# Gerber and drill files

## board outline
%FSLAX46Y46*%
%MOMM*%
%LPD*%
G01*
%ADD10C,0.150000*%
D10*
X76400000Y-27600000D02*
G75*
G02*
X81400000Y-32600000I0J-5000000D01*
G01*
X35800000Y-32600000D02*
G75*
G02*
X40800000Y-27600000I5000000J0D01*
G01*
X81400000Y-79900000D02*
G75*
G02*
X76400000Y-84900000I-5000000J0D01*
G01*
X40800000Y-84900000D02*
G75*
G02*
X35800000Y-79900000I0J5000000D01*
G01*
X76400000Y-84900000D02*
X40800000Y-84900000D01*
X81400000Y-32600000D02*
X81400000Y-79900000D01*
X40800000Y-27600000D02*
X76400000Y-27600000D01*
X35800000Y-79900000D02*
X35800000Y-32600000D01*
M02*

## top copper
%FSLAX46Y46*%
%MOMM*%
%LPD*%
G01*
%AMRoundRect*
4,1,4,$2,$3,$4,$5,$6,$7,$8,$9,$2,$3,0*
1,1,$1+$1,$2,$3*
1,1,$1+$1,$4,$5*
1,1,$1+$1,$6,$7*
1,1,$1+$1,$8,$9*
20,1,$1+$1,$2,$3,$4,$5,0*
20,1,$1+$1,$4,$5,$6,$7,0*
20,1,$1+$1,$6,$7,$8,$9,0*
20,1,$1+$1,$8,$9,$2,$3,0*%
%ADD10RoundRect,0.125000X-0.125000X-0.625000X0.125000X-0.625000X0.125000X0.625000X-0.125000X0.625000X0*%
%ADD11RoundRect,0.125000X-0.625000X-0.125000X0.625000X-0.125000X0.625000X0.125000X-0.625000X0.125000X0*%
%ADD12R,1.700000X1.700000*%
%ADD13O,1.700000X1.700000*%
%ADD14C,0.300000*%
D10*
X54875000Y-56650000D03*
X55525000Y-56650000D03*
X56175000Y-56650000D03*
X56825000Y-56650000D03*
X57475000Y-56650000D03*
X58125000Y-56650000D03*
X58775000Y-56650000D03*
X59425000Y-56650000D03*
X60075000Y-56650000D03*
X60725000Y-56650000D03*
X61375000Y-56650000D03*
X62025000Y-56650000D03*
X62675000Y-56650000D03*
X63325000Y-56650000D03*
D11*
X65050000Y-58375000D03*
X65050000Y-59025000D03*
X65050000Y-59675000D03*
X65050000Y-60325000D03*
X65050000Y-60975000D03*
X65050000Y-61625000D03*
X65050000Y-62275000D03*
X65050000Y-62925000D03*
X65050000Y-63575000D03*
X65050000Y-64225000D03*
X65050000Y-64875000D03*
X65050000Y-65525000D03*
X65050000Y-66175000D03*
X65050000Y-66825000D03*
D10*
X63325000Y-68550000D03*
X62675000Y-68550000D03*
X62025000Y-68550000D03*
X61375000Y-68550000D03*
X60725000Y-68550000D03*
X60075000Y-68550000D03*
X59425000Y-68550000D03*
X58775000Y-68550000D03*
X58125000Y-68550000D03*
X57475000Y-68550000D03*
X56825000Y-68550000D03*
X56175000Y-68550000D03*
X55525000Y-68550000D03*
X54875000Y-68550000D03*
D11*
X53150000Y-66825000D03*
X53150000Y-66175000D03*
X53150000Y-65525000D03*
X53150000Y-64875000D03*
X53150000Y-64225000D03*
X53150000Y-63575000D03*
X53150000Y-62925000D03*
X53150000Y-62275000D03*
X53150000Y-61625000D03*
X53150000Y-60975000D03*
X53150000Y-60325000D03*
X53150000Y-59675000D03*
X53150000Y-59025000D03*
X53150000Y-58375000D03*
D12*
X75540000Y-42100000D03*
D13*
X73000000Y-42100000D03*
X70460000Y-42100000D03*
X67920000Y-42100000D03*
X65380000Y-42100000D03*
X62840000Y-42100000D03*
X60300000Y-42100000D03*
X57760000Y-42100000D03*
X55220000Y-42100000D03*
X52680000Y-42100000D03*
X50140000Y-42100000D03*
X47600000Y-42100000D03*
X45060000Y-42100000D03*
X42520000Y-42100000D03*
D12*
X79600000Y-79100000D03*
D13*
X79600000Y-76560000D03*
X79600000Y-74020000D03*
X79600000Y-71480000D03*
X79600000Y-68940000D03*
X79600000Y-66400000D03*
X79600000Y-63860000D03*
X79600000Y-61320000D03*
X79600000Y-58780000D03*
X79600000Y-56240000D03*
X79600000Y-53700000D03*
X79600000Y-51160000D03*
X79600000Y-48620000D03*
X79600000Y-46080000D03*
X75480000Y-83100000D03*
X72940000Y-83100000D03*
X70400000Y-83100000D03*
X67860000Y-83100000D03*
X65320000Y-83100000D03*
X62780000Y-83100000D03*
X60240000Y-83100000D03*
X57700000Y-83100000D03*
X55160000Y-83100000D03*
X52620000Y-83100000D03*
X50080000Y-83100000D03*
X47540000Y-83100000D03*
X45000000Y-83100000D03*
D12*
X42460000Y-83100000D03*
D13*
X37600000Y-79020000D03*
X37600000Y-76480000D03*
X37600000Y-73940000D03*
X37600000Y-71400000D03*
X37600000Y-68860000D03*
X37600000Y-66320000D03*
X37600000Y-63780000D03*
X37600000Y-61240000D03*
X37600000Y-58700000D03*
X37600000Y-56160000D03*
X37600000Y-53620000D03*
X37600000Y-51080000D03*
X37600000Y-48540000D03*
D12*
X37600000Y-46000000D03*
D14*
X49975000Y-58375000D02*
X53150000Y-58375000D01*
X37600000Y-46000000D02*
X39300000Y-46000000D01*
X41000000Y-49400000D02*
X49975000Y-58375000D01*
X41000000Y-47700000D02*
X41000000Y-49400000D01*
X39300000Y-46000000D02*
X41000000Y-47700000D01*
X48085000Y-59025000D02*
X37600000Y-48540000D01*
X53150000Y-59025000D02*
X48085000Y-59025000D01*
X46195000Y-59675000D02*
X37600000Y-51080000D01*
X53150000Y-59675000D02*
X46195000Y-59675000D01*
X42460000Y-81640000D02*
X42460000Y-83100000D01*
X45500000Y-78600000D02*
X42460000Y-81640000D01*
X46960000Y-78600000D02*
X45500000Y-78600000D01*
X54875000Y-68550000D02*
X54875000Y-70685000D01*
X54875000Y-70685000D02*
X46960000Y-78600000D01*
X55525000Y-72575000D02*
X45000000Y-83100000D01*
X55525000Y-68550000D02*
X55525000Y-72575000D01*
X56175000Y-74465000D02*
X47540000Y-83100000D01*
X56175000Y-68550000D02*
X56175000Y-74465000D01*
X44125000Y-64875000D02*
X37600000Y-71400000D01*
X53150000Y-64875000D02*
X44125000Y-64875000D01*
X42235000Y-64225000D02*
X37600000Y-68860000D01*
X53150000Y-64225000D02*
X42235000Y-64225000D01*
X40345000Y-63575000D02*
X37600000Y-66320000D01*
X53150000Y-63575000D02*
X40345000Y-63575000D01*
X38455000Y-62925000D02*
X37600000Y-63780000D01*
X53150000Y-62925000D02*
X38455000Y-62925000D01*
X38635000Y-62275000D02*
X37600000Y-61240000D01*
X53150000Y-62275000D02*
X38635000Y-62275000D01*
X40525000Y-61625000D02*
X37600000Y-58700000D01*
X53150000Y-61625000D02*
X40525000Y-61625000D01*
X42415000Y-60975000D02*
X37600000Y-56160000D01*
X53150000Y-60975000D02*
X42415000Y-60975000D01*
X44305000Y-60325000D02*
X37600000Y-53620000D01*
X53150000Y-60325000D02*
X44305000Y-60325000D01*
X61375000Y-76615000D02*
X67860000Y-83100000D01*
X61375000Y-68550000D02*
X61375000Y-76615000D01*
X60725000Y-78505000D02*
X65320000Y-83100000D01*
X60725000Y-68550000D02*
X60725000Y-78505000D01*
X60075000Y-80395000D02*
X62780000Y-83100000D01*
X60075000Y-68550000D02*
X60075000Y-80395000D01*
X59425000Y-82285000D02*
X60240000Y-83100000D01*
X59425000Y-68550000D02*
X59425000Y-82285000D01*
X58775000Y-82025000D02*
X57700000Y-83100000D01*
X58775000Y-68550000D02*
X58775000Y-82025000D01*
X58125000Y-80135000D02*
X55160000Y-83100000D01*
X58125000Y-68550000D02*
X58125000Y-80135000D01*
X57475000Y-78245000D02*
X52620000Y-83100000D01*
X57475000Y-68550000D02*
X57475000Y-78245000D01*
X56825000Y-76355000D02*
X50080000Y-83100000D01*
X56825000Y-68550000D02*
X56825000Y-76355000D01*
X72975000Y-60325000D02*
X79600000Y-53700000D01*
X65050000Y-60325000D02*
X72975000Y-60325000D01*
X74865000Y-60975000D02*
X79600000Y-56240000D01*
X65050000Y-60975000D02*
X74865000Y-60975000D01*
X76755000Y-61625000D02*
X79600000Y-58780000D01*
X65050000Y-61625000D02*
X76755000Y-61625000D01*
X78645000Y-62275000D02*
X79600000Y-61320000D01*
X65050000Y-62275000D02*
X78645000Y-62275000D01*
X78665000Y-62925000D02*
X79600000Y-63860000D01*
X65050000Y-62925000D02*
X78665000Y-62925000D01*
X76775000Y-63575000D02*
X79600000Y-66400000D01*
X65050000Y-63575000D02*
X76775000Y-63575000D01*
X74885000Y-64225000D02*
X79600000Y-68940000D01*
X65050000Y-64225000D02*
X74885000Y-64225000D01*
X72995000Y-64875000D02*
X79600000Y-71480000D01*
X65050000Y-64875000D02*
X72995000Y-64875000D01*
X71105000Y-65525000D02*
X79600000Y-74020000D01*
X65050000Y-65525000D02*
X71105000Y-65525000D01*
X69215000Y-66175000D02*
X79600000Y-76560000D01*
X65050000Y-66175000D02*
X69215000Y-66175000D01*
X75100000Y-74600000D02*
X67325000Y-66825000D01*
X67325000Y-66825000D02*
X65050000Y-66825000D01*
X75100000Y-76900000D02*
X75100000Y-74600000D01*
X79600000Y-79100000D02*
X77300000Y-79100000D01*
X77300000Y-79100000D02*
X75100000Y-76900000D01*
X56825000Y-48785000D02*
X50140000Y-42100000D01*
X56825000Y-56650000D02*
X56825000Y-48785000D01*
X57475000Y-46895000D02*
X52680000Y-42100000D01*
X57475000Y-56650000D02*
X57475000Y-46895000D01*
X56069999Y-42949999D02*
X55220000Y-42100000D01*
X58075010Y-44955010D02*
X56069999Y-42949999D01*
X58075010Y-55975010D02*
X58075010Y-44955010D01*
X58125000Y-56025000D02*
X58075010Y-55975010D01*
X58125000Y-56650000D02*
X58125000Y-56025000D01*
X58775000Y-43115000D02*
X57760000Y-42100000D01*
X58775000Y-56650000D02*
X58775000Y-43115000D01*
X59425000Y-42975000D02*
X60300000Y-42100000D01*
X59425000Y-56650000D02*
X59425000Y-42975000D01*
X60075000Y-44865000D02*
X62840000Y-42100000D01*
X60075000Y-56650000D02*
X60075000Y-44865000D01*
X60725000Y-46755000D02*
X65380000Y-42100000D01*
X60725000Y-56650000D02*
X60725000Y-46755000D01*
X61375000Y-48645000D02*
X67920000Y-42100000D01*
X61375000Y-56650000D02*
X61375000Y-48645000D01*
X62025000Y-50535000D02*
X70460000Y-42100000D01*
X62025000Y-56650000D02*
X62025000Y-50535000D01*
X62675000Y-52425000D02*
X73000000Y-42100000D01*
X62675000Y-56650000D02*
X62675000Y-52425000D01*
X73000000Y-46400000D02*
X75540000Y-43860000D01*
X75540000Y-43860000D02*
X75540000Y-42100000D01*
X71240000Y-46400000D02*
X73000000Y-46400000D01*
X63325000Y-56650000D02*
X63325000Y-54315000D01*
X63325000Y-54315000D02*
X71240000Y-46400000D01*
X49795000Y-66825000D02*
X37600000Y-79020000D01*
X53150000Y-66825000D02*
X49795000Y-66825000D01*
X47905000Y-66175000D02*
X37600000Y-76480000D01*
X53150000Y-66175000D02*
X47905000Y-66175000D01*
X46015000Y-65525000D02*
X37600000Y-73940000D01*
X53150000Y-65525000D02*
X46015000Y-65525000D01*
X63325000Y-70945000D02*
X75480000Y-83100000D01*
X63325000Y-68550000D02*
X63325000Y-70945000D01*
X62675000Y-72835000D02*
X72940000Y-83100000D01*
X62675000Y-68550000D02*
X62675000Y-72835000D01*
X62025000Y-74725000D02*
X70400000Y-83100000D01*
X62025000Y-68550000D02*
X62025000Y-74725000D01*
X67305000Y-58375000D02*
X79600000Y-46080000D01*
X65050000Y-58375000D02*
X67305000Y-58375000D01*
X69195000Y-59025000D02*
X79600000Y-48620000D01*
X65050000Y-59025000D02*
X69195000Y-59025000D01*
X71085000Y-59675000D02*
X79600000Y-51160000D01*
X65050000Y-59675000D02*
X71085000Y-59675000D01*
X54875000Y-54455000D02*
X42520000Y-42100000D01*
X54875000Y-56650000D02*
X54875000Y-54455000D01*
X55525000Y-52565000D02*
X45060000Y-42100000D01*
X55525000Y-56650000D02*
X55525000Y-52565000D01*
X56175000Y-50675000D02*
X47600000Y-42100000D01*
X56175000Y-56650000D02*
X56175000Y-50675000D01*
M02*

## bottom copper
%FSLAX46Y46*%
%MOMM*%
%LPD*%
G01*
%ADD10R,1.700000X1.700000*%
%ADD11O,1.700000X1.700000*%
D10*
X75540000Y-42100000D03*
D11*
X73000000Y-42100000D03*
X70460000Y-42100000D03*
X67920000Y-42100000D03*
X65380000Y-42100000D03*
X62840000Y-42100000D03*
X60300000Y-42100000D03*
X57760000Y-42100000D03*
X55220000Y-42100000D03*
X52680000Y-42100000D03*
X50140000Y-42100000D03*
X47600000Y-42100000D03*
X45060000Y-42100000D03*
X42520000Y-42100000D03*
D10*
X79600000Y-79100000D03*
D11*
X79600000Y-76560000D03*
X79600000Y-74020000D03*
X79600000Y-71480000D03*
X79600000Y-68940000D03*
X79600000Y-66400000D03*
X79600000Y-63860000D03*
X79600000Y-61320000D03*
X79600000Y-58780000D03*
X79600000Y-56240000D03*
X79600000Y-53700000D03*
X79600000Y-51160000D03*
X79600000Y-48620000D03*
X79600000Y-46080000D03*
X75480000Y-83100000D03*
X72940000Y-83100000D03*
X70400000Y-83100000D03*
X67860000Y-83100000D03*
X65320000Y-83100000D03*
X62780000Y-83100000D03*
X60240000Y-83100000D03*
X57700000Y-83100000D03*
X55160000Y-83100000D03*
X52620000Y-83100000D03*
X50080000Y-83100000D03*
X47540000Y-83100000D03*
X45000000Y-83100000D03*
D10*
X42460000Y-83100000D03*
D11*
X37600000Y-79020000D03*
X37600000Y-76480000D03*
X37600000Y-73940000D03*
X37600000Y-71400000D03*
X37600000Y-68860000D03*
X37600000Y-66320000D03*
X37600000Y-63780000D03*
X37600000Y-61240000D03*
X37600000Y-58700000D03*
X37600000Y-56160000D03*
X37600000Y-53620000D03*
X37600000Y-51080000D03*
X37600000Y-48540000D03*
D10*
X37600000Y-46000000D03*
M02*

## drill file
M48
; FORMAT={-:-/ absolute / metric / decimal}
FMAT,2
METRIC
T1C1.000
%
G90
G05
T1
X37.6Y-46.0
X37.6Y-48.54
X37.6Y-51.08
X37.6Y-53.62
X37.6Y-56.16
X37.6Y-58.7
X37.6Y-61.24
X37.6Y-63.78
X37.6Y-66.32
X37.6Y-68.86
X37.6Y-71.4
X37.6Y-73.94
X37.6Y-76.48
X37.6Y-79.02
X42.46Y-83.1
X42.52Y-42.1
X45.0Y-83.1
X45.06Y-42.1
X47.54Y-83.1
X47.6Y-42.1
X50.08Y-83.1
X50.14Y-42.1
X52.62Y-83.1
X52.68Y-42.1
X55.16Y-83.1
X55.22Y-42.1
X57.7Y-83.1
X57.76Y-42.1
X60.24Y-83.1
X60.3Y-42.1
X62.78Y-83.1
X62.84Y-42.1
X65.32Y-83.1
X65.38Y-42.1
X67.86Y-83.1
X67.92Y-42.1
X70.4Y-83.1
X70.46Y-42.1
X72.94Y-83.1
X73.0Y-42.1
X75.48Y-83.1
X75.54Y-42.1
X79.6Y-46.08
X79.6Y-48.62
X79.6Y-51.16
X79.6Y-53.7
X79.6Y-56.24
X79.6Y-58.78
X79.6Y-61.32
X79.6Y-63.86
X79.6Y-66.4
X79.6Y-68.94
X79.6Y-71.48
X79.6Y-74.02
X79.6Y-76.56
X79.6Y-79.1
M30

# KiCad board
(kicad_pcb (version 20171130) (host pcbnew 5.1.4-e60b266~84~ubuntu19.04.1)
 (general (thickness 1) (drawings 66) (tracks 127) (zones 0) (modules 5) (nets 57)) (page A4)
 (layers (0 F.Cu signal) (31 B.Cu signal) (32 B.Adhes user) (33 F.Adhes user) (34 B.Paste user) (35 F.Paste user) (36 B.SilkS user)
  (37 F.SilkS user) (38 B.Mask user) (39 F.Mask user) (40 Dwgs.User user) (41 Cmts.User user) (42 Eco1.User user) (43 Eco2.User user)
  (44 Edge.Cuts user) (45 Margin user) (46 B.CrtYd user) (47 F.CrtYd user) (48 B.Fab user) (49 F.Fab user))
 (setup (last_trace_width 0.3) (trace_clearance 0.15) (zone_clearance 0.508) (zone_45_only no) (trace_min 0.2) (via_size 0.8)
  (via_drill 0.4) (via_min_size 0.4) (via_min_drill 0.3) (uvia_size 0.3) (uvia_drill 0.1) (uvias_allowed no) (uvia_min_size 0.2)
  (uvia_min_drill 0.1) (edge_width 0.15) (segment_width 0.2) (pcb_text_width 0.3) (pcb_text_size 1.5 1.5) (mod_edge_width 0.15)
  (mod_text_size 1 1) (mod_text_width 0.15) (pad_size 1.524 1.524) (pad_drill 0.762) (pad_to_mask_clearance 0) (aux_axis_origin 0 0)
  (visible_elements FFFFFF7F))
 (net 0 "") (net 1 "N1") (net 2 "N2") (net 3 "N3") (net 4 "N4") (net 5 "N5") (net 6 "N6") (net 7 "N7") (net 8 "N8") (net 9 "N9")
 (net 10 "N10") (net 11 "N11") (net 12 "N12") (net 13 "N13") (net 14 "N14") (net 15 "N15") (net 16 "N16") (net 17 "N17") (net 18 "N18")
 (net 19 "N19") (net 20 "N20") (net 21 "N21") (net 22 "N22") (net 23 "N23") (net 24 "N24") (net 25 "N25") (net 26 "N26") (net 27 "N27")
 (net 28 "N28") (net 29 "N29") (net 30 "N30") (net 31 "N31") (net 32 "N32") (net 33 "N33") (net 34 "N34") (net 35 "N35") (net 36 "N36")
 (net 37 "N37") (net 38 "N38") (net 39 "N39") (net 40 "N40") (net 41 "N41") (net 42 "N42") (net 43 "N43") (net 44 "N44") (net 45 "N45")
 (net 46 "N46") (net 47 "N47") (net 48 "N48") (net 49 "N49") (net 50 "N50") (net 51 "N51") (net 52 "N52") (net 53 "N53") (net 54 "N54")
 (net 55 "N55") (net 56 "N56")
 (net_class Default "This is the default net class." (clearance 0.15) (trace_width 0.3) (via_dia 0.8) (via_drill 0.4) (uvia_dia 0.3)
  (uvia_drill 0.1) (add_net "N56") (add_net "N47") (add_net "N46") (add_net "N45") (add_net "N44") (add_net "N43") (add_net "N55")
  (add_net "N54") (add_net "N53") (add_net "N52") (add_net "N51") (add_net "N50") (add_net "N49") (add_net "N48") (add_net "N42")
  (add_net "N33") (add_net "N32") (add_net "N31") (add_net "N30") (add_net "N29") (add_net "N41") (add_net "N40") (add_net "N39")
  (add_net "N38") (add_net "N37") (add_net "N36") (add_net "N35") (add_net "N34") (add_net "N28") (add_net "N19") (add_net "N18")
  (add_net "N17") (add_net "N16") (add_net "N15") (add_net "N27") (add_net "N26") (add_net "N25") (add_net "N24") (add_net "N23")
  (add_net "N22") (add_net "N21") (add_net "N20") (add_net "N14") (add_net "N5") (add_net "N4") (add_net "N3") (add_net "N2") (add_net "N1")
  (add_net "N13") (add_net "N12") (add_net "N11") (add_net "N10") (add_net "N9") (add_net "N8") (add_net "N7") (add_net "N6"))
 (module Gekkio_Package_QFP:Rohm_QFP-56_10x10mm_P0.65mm (layer F.Cu) (at 59.1 62.6)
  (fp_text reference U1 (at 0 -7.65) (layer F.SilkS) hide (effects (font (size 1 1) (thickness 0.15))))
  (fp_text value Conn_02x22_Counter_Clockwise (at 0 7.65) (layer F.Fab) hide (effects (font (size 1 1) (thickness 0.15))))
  (pad 56 smd roundrect (at -4.225 -5.95) (size 0.5 1.5) (layers F.Cu F.Paste F.Mask) (roundrect_rratio 0.25) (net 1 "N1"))
  (pad 55 smd roundrect (at -3.575 -5.95) (size 0.5 1.5) (layers F.Cu F.Paste F.Mask) (roundrect_rratio 0.25) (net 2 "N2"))
  (pad 54 smd roundrect (at -2.925 -5.95) (size 0.5 1.5) (layers F.Cu F.Paste F.Mask) (roundrect_rratio 0.25) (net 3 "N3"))
  (pad 53 smd roundrect (at -2.275 -5.95) (size 0.5 1.5) (layers F.Cu F.Paste F.Mask) (roundrect_rratio 0.25) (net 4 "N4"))
  (pad 52 smd roundrect (at -1.625 -5.95) (size 0.5 1.5) (layers F.Cu F.Paste F.Mask) (roundrect_rratio 0.25) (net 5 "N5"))
  (pad 51 smd roundrect (at -0.975 -5.95) (size 0.5 1.5) (layers F.Cu F.Paste F.Mask) (roundrect_rratio 0.25) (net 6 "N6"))
  (pad 50 smd roundrect (at -0.325 -5.95) (size 0.5 1.5) (layers F.Cu F.Paste F.Mask) (roundrect_rratio 0.25) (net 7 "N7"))
  (pad 49 smd roundrect (at 0.325 -5.95) (size 0.5 1.5) (layers F.Cu F.Paste F.Mask) (roundrect_rratio 0.25) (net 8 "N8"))
  (pad 48 smd roundrect (at 0.975 -5.95) (size 0.5 1.5) (layers F.Cu F.Paste F.Mask) (roundrect_rratio 0.25) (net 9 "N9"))
  (pad 47 smd roundrect (at 1.625 -5.95) (size 0.5 1.5) (layers F.Cu F.Paste F.Mask) (roundrect_rratio 0.25) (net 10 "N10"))
  (pad 46 smd roundrect (at 2.275 -5.95) (size 0.5 1.5) (layers F.Cu F.Paste F.Mask) (roundrect_rratio 0.25) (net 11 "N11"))
  (pad 45 smd roundrect (at 2.925 -5.95) (size 0.5 1.5) (layers F.Cu F.Paste F.Mask) (roundrect_rratio 0.25) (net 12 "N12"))
  (pad 44 smd roundrect (at 3.575 -5.95) (size 0.5 1.5) (layers F.Cu F.Paste F.Mask) (roundrect_rratio 0.25) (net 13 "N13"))
  (pad 43 smd roundrect (at 4.225 -5.95) (size 0.5 1.5) (layers F.Cu F.Paste F.Mask) (roundrect_rratio 0.25) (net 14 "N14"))
  (pad 42 smd roundrect (at 5.95 -4.225) (size 1.5 0.5) (layers F.Cu F.Paste F.Mask) (roundrect_rratio 0.25) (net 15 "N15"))
  (pad 41 smd roundrect (at 5.95 -3.575) (size 1.5 0.5) (layers F.Cu F.Paste F.Mask) (roundrect_rratio 0.25) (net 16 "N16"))
  (pad 40 smd roundrect (at 5.95 -2.925) (size 1.5 0.5) (layers F.Cu F.Paste F.Mask) (roundrect_rratio 0.25) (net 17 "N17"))
  (pad 39 smd roundrect (at 5.95 -2.275) (size 1.5 0.5) (layers F.Cu F.Paste F.Mask) (roundrect_rratio 0.25) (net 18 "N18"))
  (pad 38 smd roundrect (at 5.95 -1.625) (size 1.5 0.5) (layers F.Cu F.Paste F.Mask) (roundrect_rratio 0.25) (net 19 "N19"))
  (pad 37 smd roundrect (at 5.95 -0.975) (size 1.5 0.5) (layers F.Cu F.Paste F.Mask) (roundrect_rratio 0.25) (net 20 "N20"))
  (pad 36 smd roundrect (at 5.95 -0.325) (size 1.5 0.5) (layers F.Cu F.Paste F.Mask) (roundrect_rratio 0.25) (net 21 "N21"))
  (pad 35 smd roundrect (at 5.95 0.325) (size 1.5 0.5) (layers F.Cu F.Paste F.Mask) (roundrect_rratio 0.25) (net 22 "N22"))
  (pad 34 smd roundrect (at 5.95 0.975) (size 1.5 0.5) (layers F.Cu F.Paste F.Mask) (roundrect_rratio 0.25) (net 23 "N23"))
  (pad 33 smd roundrect (at 5.95 1.625) (size 1.5 0.5) (layers F.Cu F.Paste F.Mask) (roundrect_rratio 0.25) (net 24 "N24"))
  (pad 32 smd roundrect (at 5.95 2.275) (size 1.5 0.5) (layers F.Cu F.Paste F.Mask) (roundrect_rratio 0.25) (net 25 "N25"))
  (pad 31 smd roundrect (at 5.95 2.925) (size 1.5 0.5) (layers F.Cu F.Paste F.Mask) (roundrect_rratio 0.25) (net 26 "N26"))
  (pad 30 smd roundrect (at 5.95 3.575) (size 1.5 0.5) (layers F.Cu F.Paste F.Mask) (roundrect_rratio 0.25) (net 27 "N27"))
  (pad 29 smd roundrect (at 5.95 4.225) (size 1.5 0.5) (layers F.Cu F.Paste F.Mask) (roundrect_rratio 0.25) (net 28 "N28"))
  (pad 28 smd roundrect (at 4.225 5.95) (size 0.5 1.5) (layers F.Cu F.Paste F.Mask) (roundrect_rratio 0.25) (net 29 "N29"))
  (pad 27 smd roundrect (at 3.575 5.95) (size 0.5 1.5) (layers F.Cu F.Paste F.Mask) (roundrect_rratio 0.25) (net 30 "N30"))
  (pad 26 smd roundrect (at 2.925 5.95) (size 0.5 1.5) (layers F.Cu F.Paste F.Mask) (roundrect_rratio 0.25) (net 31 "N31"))
  (pad 25 smd roundrect (at 2.275 5.95) (size 0.5 1.5) (layers F.Cu F.Paste F.Mask) (roundrect_rratio 0.25) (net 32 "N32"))
  (pad 24 smd roundrect (at 1.625 5.95) (size 0.5 1.5) (layers F.Cu F.Paste F.Mask) (roundrect_rratio 0.25) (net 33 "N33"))
  (pad 23 smd roundrect (at 0.975 5.95) (size 0.5 1.5) (layers F.Cu F.Paste F.Mask) (roundrect_rratio 0.25) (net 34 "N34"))
  (pad 22 smd roundrect (at 0.325 5.95) (size 0.5 1.5) (layers F.Cu F.Paste F.Mask) (roundrect_rratio 0.25) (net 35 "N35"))
  (pad 21 smd roundrect (at -0.325 5.95) (size 0.5 1.5) (layers F.Cu F.Paste F.Mask) (roundrect_rratio 0.25) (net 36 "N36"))
  (pad 20 smd roundrect (at -0.975 5.95) (size 0.5 1.5) (layers F.Cu F.Paste F.Mask) (roundrect_rratio 0.25) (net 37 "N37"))
  (pad 19 smd roundrect (at -1.625 5.95) (size 0.5 1.5) (layers F.Cu F.Paste F.Mask) (roundrect_rratio 0.25) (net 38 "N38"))
  (pad 18 smd roundrect (at -2.275 5.95) (size 0.5 1.5) (layers F.Cu F.Paste F.Mask) (roundrect_rratio 0.25) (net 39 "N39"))
  (pad 17 smd roundrect (at -2.925 5.95) (size 0.5 1.5) (layers F.Cu F.Paste F.Mask) (roundrect_rratio 0.25) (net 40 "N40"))
  (pad 16 smd roundrect (at -3.575 5.95) (size 0.5 1.5) (layers F.Cu F.Paste F.Mask) (roundrect_rratio 0.25) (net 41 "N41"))
  (pad 15 smd roundrect (at -4.225 5.95) (size 0.5 1.5) (layers F.Cu F.Paste F.Mask) (roundrect_rratio 0.25) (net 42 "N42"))
  (pad 14 smd roundrect (at -5.95 4.225) (size 1.5 0.5) (layers F.Cu F.Paste F.Mask) (roundrect_rratio 0.25) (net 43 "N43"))
  (pad 13 smd roundrect (at -5.95 3.575) (size 1.5 0.5) (layers F.Cu F.Paste F.Mask) (roundrect_rratio 0.25) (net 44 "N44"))
  (pad 12 smd roundrect (at -5.95 2.925) (size 1.5 0.5) (layers F.Cu F.Paste F.Mask) (roundrect_rratio 0.25) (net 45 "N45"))
  (pad 11 smd roundrect (at -5.95 2.275) (size 1.5 0.5) (layers F.Cu F.Paste F.Mask) (roundrect_rratio 0.25) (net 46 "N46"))
  (pad 10 smd roundrect (at -5.95 1.625) (size 1.5 0.5) (layers F.Cu F.Paste F.Mask) (roundrect_rratio 0.25) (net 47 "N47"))
  (pad 9 smd roundrect (at -5.95 0.975) (size 1.5 0.5) (layers F.Cu F.Paste F.Mask) (roundrect_rratio 0.25) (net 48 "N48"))
  (pad 8 smd roundrect (at -5.95 0.325) (size 1.5 0.5) (layers F.Cu F.Paste F.Mask) (roundrect_rratio 0.25) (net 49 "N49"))
  (pad 7 smd roundrect (at -5.95 -0.325) (size 1.5 0.5) (layers F.Cu F.Paste F.Mask) (roundrect_rratio 0.25) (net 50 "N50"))
  (pad 6 smd roundrect (at -5.95 -0.975) (size 1.5 0.5) (layers F.Cu F.Paste F.Mask) (roundrect_rratio 0.25) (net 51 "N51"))
  (pad 5 smd roundrect (at -5.95 -1.625) (size 1.5 0.5) (layers F.Cu F.Paste F.Mask) (roundrect_rratio 0.25) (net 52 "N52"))
  (pad 4 smd roundrect (at -5.95 -2.275) (size 1.5 0.5) (layers F.Cu F.Paste F.Mask) (roundrect_rratio 0.25) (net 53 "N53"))
  (pad 3 smd roundrect (at -5.95 -2.925) (size 1.5 0.5) (layers F.Cu F.Paste F.Mask) (roundrect_rratio 0.25) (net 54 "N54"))
  (pad 2 smd roundrect (at -5.95 -3.575) (size 1.5 0.5) (layers F.Cu F.Paste F.Mask) (roundrect_rratio 0.25) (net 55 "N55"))
  (pad 1 smd roundrect (at -5.95 -4.225) (size 1.5 0.5) (layers F.Cu F.Paste F.Mask) (roundrect_rratio 0.25) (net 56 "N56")))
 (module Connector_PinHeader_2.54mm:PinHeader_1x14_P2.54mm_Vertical (layer F.Cu) (at 75.54 42.1 270)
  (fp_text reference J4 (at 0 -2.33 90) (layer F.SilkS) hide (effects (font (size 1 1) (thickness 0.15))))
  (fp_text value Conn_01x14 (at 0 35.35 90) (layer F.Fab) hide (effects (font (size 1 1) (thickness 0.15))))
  (pad 1 thru_hole rect (at 0 0 270) (size 1.7 1.7) (drill 1) (layers *.Cu *.Mask) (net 14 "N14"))
  (pad 2 thru_hole oval (at 0 2.54 270) (size 1.7 1.7) (drill 1) (layers *.Cu *.Mask) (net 13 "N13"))
  (pad 3 thru_hole oval (at 0 5.08 270) (size 1.7 1.7) (drill 1) (layers *.Cu *.Mask) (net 12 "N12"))
  (pad 4 thru_hole oval (at 0 7.62 270) (size 1.7 1.7) (drill 1) (layers *.Cu *.Mask) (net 11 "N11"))
  (pad 5 thru_hole oval (at 0 10.16 270) (size 1.7 1.7) (drill 1) (layers *.Cu *.Mask) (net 10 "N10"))
  (pad 6 thru_hole oval (at 0 12.7 270) (size 1.7 1.7) (drill 1) (layers *.Cu *.Mask) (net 9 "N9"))
  (pad 7 thru_hole oval (at 0 15.24 270) (size 1.7 1.7) (drill 1) (layers *.Cu *.Mask) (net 8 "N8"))
  (pad 8 thru_hole oval (at 0 17.78 270) (size 1.7 1.7) (drill 1) (layers *.Cu *.Mask) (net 7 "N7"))
  (pad 9 thru_hole oval (at 0 20.32 270) (size 1.7 1.7) (drill 1) (layers *.Cu *.Mask) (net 6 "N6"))
  (pad 10 thru_hole oval (at 0 22.86 270) (size 1.7 1.7) (drill 1) (layers *.Cu *.Mask) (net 5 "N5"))
  (pad 11 thru_hole oval (at 0 25.4 270) (size 1.7 1.7) (drill 1) (layers *.Cu *.Mask) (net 4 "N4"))
  (pad 12 thru_hole oval (at 0 27.94 270) (size 1.7 1.7) (drill 1) (layers *.Cu *.Mask) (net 3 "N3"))
  (pad 13 thru_hole oval (at 0 30.48 270) (size 1.7 1.7) (drill 1) (layers *.Cu *.Mask) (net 2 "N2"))
  (pad 14 thru_hole oval (at 0 33.02 270) (size 1.7 1.7) (drill 1) (layers *.Cu *.Mask) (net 1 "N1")))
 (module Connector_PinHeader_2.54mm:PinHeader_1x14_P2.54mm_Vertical (layer F.Cu) (at 79.6 79.1 180)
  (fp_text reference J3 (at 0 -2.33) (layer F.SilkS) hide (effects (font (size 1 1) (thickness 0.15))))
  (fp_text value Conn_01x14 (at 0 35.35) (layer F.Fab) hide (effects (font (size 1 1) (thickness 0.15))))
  (pad 1 thru_hole rect (at 0 0 180) (size 1.7 1.7) (drill 1) (layers *.Cu *.Mask) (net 28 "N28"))
  (pad 2 thru_hole oval (at 0 2.54 180) (size 1.7 1.7) (drill 1) (layers *.Cu *.Mask) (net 27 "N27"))
  (pad 3 thru_hole oval (at 0 5.08 180) (size 1.7 1.7) (drill 1) (layers *.Cu *.Mask) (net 26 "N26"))
  (pad 4 thru_hole oval (at 0 7.62 180) (size 1.7 1.7) (drill 1) (layers *.Cu *.Mask) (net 25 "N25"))
  (pad 5 thru_hole oval (at 0 10.16 180) (size 1.7 1.7) (drill 1) (layers *.Cu *.Mask) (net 24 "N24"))
  (pad 6 thru_hole oval (at 0 12.7 180) (size 1.7 1.7) (drill 1) (layers *.Cu *.Mask) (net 23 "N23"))
  (pad 7 thru_hole oval (at 0 15.24 180) (size 1.7 1.7) (drill 1) (layers *.Cu *.Mask) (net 22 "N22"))
  (pad 8 thru_hole oval (at 0 17.78 180) (size 1.7 1.7) (drill 1) (layers *.Cu *.Mask) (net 21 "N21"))
  (pad 9 thru_hole oval (at 0 20.32 180) (size 1.7 1.7) (drill 1) (layers *.Cu *.Mask) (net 20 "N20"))
  (pad 10 thru_hole oval (at 0 22.86 180) (size 1.7 1.7) (drill 1) (layers *.Cu *.Mask) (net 19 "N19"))
  (pad 11 thru_hole oval (at 0 25.4 180) (size 1.7 1.7) (drill 1) (layers *.Cu *.Mask) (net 18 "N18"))
  (pad 12 thru_hole oval (at 0 27.94 180) (size 1.7 1.7) (drill 1) (layers *.Cu *.Mask) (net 17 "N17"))
  (pad 13 thru_hole oval (at 0 30.48 180) (size 1.7 1.7) (drill 1) (layers *.Cu *.Mask) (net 16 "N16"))
  (pad 14 thru_hole oval (at 0 33.02 180) (size 1.7 1.7) (drill 1) (layers *.Cu *.Mask) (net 15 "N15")))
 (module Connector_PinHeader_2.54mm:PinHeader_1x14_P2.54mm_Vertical (layer F.Cu) (at 42.46 83.1 90)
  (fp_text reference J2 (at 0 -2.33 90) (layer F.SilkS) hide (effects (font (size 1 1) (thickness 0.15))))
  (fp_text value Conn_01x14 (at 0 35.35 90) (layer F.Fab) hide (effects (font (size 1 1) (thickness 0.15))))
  (pad 14 thru_hole oval (at 0 33.02 90) (size 1.7 1.7) (drill 1) (layers *.Cu *.Mask) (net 29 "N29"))
  (pad 13 thru_hole oval (at 0 30.48 90) (size 1.7 1.7) (drill 1) (layers *.Cu *.Mask) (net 30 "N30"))
  (pad 12 thru_hole oval (at 0 27.94 90) (size 1.7 1.7) (drill 1) (layers *.Cu *.Mask) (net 31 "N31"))
  (pad 11 thru_hole oval (at 0 25.4 90) (size 1.7 1.7) (drill 1) (layers *.Cu *.Mask) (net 32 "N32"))
  (pad 10 thru_hole oval (at 0 22.86 90) (size 1.7 1.7) (drill 1) (layers *.Cu *.Mask) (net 33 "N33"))
  (pad 9 thru_hole oval (at 0 20.32 90) (size 1.7 1.7) (drill 1) (layers *.Cu *.Mask) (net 34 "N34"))
  (pad 8 thru_hole oval (at 0 17.78 90) (size 1.7 1.7) (drill 1) (layers *.Cu *.Mask) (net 35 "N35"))
  (pad 7 thru_hole oval (at 0 15.24 90) (size 1.7 1.7) (drill 1) (layers *.Cu *.Mask) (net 36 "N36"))
  (pad 6 thru_hole oval (at 0 12.7 90) (size 1.7 1.7) (drill 1) (layers *.Cu *.Mask) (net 37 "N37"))
  (pad 5 thru_hole oval (at 0 10.16 90) (size 1.7 1.7) (drill 1) (layers *.Cu *.Mask) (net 38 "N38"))
  (pad 4 thru_hole oval (at 0 7.62 90) (size 1.7 1.7) (drill 1) (layers *.Cu *.Mask) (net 39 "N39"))
  (pad 3 thru_hole oval (at 0 5.08 90) (size 1.7 1.7) (drill 1) (layers *.Cu *.Mask) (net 40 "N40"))
  (pad 2 thru_hole oval (at 0 2.54 90) (size 1.7 1.7) (drill 1) (layers *.Cu *.Mask) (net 41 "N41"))
  (pad 1 thru_hole rect (at 0 0 90) (size 1.7 1.7) (drill 1) (layers *.Cu *.Mask) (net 42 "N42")))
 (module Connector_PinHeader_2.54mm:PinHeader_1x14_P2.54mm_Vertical (layer F.Cu) (at 37.6 46)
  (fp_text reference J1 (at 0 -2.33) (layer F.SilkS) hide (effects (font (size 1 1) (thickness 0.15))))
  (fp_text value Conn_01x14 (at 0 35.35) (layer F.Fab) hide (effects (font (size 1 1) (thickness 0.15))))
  (pad 14 thru_hole oval (at 0 33.02) (size 1.7 1.7) (drill 1) (layers *.Cu *.Mask) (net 43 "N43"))
  (pad 13 thru_hole oval (at 0 30.48) (size 1.7 1.7) (drill 1) (layers *.Cu *.Mask) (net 44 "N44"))
  (pad 12 thru_hole oval (at 0 27.94) (size 1.7 1.7) (drill 1) (layers *.Cu *.Mask) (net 45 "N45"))
  (pad 11 thru_hole oval (at 0 25.4) (size 1.7 1.7) (drill 1) (layers *.Cu *.Mask) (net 46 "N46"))
  (pad 10 thru_hole oval (at 0 22.86) (size 1.7 1.7) (drill 1) (layers *.Cu *.Mask) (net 47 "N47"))
  (pad 9 thru_hole oval (at 0 20.32) (size 1.7 1.7) (drill 1) (layers *.Cu *.Mask) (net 48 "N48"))
  (pad 8 thru_hole oval (at 0 17.78) (size 1.7 1.7) (drill 1) (layers *.Cu *.Mask) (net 49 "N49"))
  (pad 7 thru_hole oval (at 0 15.24) (size 1.7 1.7) (drill 1) (layers *.Cu *.Mask) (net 50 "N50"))
  (pad 6 thru_hole oval (at 0 12.7) (size 1.7 1.7) (drill 1) (layers *.Cu *.Mask) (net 51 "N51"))
  (pad 5 thru_hole oval (at 0 10.16) (size 1.7 1.7) (drill 1) (layers *.Cu *.Mask) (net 52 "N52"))
  (pad 4 thru_hole oval (at 0 7.62) (size 1.7 1.7) (drill 1) (layers *.Cu *.Mask) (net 53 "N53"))
  (pad 3 thru_hole oval (at 0 5.08) (size 1.7 1.7) (drill 1) (layers *.Cu *.Mask) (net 54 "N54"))
  (pad 2 thru_hole oval (at 0 2.54) (size 1.7 1.7) (drill 1) (layers *.Cu *.Mask) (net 55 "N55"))
  (pad 1 thru_hole rect (at 0 0) (size 1.7 1.7) (drill 1) (layers *.Cu *.Mask) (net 56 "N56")))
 (gr_arc (start 76.4 32.6) (end 81.4 32.6) (angle -90) (layer Edge.Cuts) (width 0.15))
 (gr_arc (start 40.8 32.6) (end 40.8 27.6) (angle -90) (layer Edge.Cuts) (width 0.15))
 (gr_arc (start 76.4 79.9) (end 76.4 84.9) (angle -90) (layer Edge.Cuts) (width 0.15))
 (gr_arc (start 40.8 79.9) (end 35.8 79.9) (angle -90) (layer Edge.Cuts) (width 0.15))
 (gr_line (start 76.4 84.9) (end 40.8 84.9) (layer Edge.Cuts) (width 0.15))
 (gr_line (start 81.4 32.6) (end 81.4 79.9) (layer Edge.Cuts) (width 0.15))
 (gr_line (start 40.8 27.6) (end 76.4 27.6) (layer Edge.Cuts) (width 0.15))
 (gr_line (start 35.8 79.9) (end 35.8 32.6) (layer Edge.Cuts) (width 0.15))
 (segment (start 49.975 58.375) (end 53.15 58.375) (width 0.3) (layer F.Cu) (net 56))
 (segment (start 37.6 46) (end 39.3 46) (width 0.3) (layer F.Cu) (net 56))
 (segment (start 41 49.4) (end 49.975 58.375) (width 0.3) (layer F.Cu) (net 56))
 (segment (start 41 47.7) (end 41 49.4) (width 0.3) (layer F.Cu) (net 56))
 (segment (start 39.3 46) (end 41 47.7) (width 0.3) (layer F.Cu) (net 56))
 (segment (start 48.085 59.025) (end 37.6 48.54) (width 0.3) (layer F.Cu) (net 55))
 (segment (start 53.15 59.025) (end 48.085 59.025) (width 0.3) (layer F.Cu) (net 55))
 (segment (start 46.195 59.675) (end 37.6 51.08) (width 0.3) (layer F.Cu) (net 54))
 (segment (start 53.15 59.675) (end 46.195 59.675) (width 0.3) (layer F.Cu) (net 54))
 (segment (start 42.46 81.64) (end 42.46 83.1) (width 0.3) (layer F.Cu) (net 42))
 (segment (start 45.5 78.6) (end 42.46 81.64) (width 0.3) (layer F.Cu) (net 42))
 (segment (start 46.96 78.6) (end 45.5 78.6) (width 0.3) (layer F.Cu) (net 42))
 (segment (start 54.875 68.55) (end 54.875 70.685) (width 0.3) (layer F.Cu) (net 42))
 (segment (start 54.875 70.685) (end 46.96 78.6) (width 0.3) (layer F.Cu) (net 42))
 (segment (start 55.525 72.575) (end 45 83.1) (width 0.3) (layer F.Cu) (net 41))
 (segment (start 55.525 68.55) (end 55.525 72.575) (width 0.3) (layer F.Cu) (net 41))
 (segment (start 56.175 74.465) (end 47.54 83.1) (width 0.3) (layer F.Cu) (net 40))
 (segment (start 56.175 68.55) (end 56.175 74.465) (width 0.3) (layer F.Cu) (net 40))
 (segment (start 44.125 64.875) (end 37.6 71.4) (width 0.3) (layer F.Cu) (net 46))
 (segment (start 53.15 64.875) (end 44.125 64.875) (width 0.3) (layer F.Cu) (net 46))
 (segment (start 42.235 64.225) (end 37.6 68.86) (width 0.3) (layer F.Cu) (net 47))
 (segment (start 53.15 64.225) (end 42.235 64.225) (width 0.3) (layer F.Cu) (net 47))
 (segment (start 40.345 63.575) (end 37.6 66.32) (width 0.3) (layer F.Cu) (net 48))
 (segment (start 53.15 63.575) (end 40.345 63.575) (width 0.3) (layer F.Cu) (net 48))
 (segment (start 38.455 62.925) (end 37.6 63.78) (width 0.3) (layer F.Cu) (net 49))
 (segment (start 53.15 62.925) (end 38.455 62.925) (width 0.3) (layer F.Cu) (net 49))
 (segment (start 38.635 62.275) (end 37.6 61.24) (width 0.3) (layer F.Cu) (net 50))
 (segment (start 53.15 62.275) (end 38.635 62.275) (width 0.3) (layer F.Cu) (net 50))
 (segment (start 40.525 61.625) (end 37.6 58.7) (width 0.3) (layer F.Cu) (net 51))
 (segment (start 53.15 61.625) (end 40.525 61.625) (width 0.3) (layer F.Cu) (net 51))
 (segment (start 42.415 60.975) (end 37.6 56.16) (width 0.3) (layer F.Cu) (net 52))
 (segment (start 53.15 60.975) (end 42.415 60.975) (width 0.3) (layer F.Cu) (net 52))
 (segment (start 44.305 60.325) (end 37.6 53.62) (width 0.3) (layer F.Cu) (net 53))
 (segment (start 53.15 60.325) (end 44.305 60.325) (width 0.3) (layer F.Cu) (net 53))
 (segment (start 61.375 76.615) (end 67.86 83.1) (width 0.3) (layer F.Cu) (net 32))
 (segment (start 61.375 68.55) (end 61.375 76.615) (width 0.3) (layer F.Cu) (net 32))
 (segment (start 60.725 78.505) (end 65.32 83.1) (width 0.3) (layer F.Cu) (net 33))
 (segment (start 60.725 68.55) (end 60.725 78.505) (width 0.3) (layer F.Cu) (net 33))
 (segment (start 60.075 80.395) (end 62.78 83.1) (width 0.3) (layer F.Cu) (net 34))
 (segment (start 60.075 68.55) (end 60.075 80.395) (width 0.3) (layer F.Cu) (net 34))
 (segment (start 59.425 82.285) (end 60.24 83.1) (width 0.3) (layer F.Cu) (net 35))
 (segment (start 59.425 68.55) (end 59.425 82.285) (width 0.3) (layer F.Cu) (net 35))
 (segment (start 58.775 82.025) (end 57.7 83.1) (width 0.3) (layer F.Cu) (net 36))
 (segment (start 58.775 68.55) (end 58.775 82.025) (width 0.3) (layer F.Cu) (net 36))
 (segment (start 58.125 80.135) (end 55.16 83.1) (width 0.3) (layer F.Cu) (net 37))
 (segment (start 58.125 68.55) (end 58.125 80.135) (width 0.3) (layer F.Cu) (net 37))
 (segment (start 57.475 78.245) (end 52.62 83.1) (width 0.3) (layer F.Cu) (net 38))
 (segment (start 57.475 68.55) (end 57.475 78.245) (width 0.3) (layer F.Cu) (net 38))
 (segment (start 56.825 76.355) (end 50.08 83.1) (width 0.3) (layer F.Cu) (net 39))
 (segment (start 56.825 68.55) (end 56.825 76.355) (width 0.3) (layer F.Cu) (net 39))
 (segment (start 72.975 60.325) (end 79.6 53.7) (width 0.3) (layer F.Cu) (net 18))
 (segment (start 65.05 60.325) (end 72.975 60.325) (width 0.3) (layer F.Cu) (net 18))
 (segment (start 74.865 60.975) (end 79.6 56.24) (width 0.3) (layer F.Cu) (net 19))
 (segment (start 65.05 60.975) (end 74.865 60.975) (width 0.3) (layer F.Cu) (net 19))
 (segment (start 76.755 61.625) (end 79.6 58.78) (width 0.3) (layer F.Cu) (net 20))
 (segment (start 65.05 61.625) (end 76.755 61.625) (width 0.3) (layer F.Cu) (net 20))
 (segment (start 78.645 62.275) (end 79.6 61.32) (width 0.3) (layer F.Cu) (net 21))
 (segment (start 65.05 62.275) (end 78.645 62.275) (width 0.3) (layer F.Cu) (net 21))
 (segment (start 78.665 62.925) (end 79.6 63.86) (width 0.3) (layer F.Cu) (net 22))
 (segment (start 65.05 62.925) (end 78.665 62.925) (width 0.3) (layer F.Cu) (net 22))
 (segment (start 76.775 63.575) (end 79.6 66.4) (width 0.3) (layer F.Cu) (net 23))
 (segment (start 65.05 63.575) (end 76.775 63.575) (width 0.3) (layer F.Cu) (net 23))
 (segment (start 74.885 64.225) (end 79.6 68.94) (width 0.3) (layer F.Cu) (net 24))
 (segment (start 65.05 64.225) (end 74.885 64.225) (width 0.3) (layer F.Cu) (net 24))
 (segment (start 72.995 64.875) (end 79.6 71.48) (width 0.3) (layer F.Cu) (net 25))
 (segment (start 65.05 64.875) (end 72.995 64.875) (width 0.3) (layer F.Cu) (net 25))
 (segment (start 71.105 65.525) (end 79.6 74.02) (width 0.3) (layer F.Cu) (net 26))
 (segment (start 65.05 65.525) (end 71.105 65.525) (width 0.3) (layer F.Cu) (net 26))
 (segment (start 69.215 66.175) (end 79.6 76.56) (width 0.3) (layer F.Cu) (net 27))
 (segment (start 65.05 66.175) (end 69.215 66.175) (width 0.3) (layer F.Cu) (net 27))
 (segment (start 75.1 74.6) (end 67.325 66.825) (width 0.3) (layer F.Cu) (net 28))
 (segment (start 67.325 66.825) (end 65.05 66.825) (width 0.3) (layer F.Cu) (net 28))
 (segment (start 75.1 76.9) (end 75.1 74.6) (width 0.3) (layer F.Cu) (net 28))
 (segment (start 79.6 79.1) (end 77.3 79.1) (width 0.3) (layer F.Cu) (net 28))
 (segment (start 77.3 79.1) (end 75.1 76.9) (width 0.3) (layer F.Cu) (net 28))
 (segment (start 56.825 48.785) (end 50.14 42.1) (width 0.3) (layer F.Cu) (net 4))
 (segment (start 56.825 56.65) (end 56.825 48.785) (width 0.3) (layer F.Cu) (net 4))
 (segment (start 57.475 46.895) (end 52.68 42.1) (width 0.3) (layer F.Cu) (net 5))
 (segment (start 57.475 56.65) (end 57.475 46.895) (width 0.3) (layer F.Cu) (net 5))
 (segment (start 56.069999 42.949999) (end 55.22 42.1) (width 0.3) (layer F.Cu) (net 6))
 (segment (start 58.07501 44.95501) (end 56.069999 42.949999) (width 0.3) (layer F.Cu) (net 6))
 (segment (start 58.07501 55.97501) (end 58.07501 44.95501) (width 0.3) (layer F.Cu) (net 6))
 (segment (start 58.125 56.025) (end 58.07501 55.97501) (width 0.3) (layer F.Cu) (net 6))
 (segment (start 58.125 56.65) (end 58.125 56.025) (width 0.3) (layer F.Cu) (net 6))
 (segment (start 58.775 43.115) (end 57.76 42.1) (width 0.3) (layer F.Cu) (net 7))
 (segment (start 58.775 56.65) (end 58.775 43.115) (width 0.3) (layer F.Cu) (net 7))
 (segment (start 59.425 42.975) (end 60.3 42.1) (width 0.3) (layer F.Cu) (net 8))
 (segment (start 59.425 56.65) (end 59.425 42.975) (width 0.3) (layer F.Cu) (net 8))
 (segment (start 60.075 44.865) (end 62.84 42.1) (width 0.3) (layer F.Cu) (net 9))
 (segment (start 60.075 56.65) (end 60.075 44.865) (width 0.3) (layer F.Cu) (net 9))
 (segment (start 60.725 46.755) (end 65.38 42.1) (width 0.3) (layer F.Cu) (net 10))
 (segment (start 60.725 56.65) (end 60.725 46.755) (width 0.3) (layer F.Cu) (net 10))
 (segment (start 61.375 48.645) (end 67.92 42.1) (width 0.3) (layer F.Cu) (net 11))
 (segment (start 61.375 56.65) (end 61.375 48.645) (width 0.3) (layer F.Cu) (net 11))
 (segment (start 62.025 50.535) (end 70.46 42.1) (width 0.3) (layer F.Cu) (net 12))
 (segment (start 62.025 56.65) (end 62.025 50.535) (width 0.3) (layer F.Cu) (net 12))
 (segment (start 62.675 52.425) (end 73 42.1) (width 0.3) (layer F.Cu) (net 13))
 (segment (start 62.675 56.65) (end 62.675 52.425) (width 0.3) (layer F.Cu) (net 13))
 (segment (start 73 46.4) (end 75.54 43.86) (width 0.3) (layer F.Cu) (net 14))
 (segment (start 75.54 43.86) (end 75.54 42.1) (width 0.3) (layer F.Cu) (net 14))
 (segment (start 71.24 46.4) (end 73 46.4) (width 0.3) (layer F.Cu) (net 14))
 (segment (start 63.325 56.65) (end 63.325 54.315) (width 0.3) (layer F.Cu) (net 14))
 (segment (start 63.325 54.315) (end 71.24 46.4) (width 0.3) (layer F.Cu) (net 14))
 (segment (start 49.795 66.825) (end 37.6 79.02) (width 0.3) (layer F.Cu) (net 43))
 (segment (start 53.15 66.825) (end 49.795 66.825) (width 0.3) (layer F.Cu) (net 43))
 (segment (start 47.905 66.175) (end 37.6 76.48) (width 0.3) (layer F.Cu) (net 44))
 (segment (start 53.15 66.175) (end 47.905 66.175) (width 0.3) (layer F.Cu) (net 44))
 (segment (start 46.015 65.525) (end 37.6 73.94) (width 0.3) (layer F.Cu) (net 45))
 (segment (start 53.15 65.525) (end 46.015 65.525) (width 0.3) (layer F.Cu) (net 45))
 (segment (start 63.325 70.945) (end 75.48 83.1) (width 0.3) (layer F.Cu) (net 29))
 (segment (start 63.325 68.55) (end 63.325 70.945) (width 0.3) (layer F.Cu) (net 29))
 (segment (start 62.675 72.835) (end 72.94 83.1) (width 0.3) (layer F.Cu) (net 30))
 (segment (start 62.675 68.55) (end 62.675 72.835) (width 0.3) (layer F.Cu) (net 30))
 (segment (start 62.025 74.725) (end 70.4 83.1) (width 0.3) (layer F.Cu) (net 31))
 (segment (start 62.025 68.55) (end 62.025 74.725) (width 0.3) (layer F.Cu) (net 31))
 (segment (start 67.305 58.375) (end 79.6 46.08) (width 0.3) (layer F.Cu) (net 15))
 (segment (start 65.05 58.375) (end 67.305 58.375) (width 0.3) (layer F.Cu) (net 15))
 (segment (start 69.195 59.025) (end 79.6 48.62) (width 0.3) (layer F.Cu) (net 16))
 (segment (start 65.05 59.025) (end 69.195 59.025) (width 0.3) (layer F.Cu) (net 16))
 (segment (start 71.085 59.675) (end 79.6 51.16) (width 0.3) (layer F.Cu) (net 17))
 (segment (start 65.05 59.675) (end 71.085 59.675) (width 0.3) (layer F.Cu) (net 17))
 (segment (start 54.875 54.455) (end 42.52 42.1) (width 0.3) (layer F.Cu) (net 1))
 (segment (start 54.875 56.65) (end 54.875 54.455) (width 0.3) (layer F.Cu) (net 1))
 (segment (start 55.525 52.565) (end 45.06 42.1) (width 0.3) (layer F.Cu) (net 2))
 (segment (start 55.525 56.65) (end 55.525 52.565) (width 0.3) (layer F.Cu) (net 2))
 (segment (start 56.175 50.675) (end 47.6 42.1) (width 0.3) (layer F.Cu) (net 3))
 (segment (start 56.175 56.65) (end 56.175 50.675) (width 0.3) (layer F.Cu) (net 3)))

